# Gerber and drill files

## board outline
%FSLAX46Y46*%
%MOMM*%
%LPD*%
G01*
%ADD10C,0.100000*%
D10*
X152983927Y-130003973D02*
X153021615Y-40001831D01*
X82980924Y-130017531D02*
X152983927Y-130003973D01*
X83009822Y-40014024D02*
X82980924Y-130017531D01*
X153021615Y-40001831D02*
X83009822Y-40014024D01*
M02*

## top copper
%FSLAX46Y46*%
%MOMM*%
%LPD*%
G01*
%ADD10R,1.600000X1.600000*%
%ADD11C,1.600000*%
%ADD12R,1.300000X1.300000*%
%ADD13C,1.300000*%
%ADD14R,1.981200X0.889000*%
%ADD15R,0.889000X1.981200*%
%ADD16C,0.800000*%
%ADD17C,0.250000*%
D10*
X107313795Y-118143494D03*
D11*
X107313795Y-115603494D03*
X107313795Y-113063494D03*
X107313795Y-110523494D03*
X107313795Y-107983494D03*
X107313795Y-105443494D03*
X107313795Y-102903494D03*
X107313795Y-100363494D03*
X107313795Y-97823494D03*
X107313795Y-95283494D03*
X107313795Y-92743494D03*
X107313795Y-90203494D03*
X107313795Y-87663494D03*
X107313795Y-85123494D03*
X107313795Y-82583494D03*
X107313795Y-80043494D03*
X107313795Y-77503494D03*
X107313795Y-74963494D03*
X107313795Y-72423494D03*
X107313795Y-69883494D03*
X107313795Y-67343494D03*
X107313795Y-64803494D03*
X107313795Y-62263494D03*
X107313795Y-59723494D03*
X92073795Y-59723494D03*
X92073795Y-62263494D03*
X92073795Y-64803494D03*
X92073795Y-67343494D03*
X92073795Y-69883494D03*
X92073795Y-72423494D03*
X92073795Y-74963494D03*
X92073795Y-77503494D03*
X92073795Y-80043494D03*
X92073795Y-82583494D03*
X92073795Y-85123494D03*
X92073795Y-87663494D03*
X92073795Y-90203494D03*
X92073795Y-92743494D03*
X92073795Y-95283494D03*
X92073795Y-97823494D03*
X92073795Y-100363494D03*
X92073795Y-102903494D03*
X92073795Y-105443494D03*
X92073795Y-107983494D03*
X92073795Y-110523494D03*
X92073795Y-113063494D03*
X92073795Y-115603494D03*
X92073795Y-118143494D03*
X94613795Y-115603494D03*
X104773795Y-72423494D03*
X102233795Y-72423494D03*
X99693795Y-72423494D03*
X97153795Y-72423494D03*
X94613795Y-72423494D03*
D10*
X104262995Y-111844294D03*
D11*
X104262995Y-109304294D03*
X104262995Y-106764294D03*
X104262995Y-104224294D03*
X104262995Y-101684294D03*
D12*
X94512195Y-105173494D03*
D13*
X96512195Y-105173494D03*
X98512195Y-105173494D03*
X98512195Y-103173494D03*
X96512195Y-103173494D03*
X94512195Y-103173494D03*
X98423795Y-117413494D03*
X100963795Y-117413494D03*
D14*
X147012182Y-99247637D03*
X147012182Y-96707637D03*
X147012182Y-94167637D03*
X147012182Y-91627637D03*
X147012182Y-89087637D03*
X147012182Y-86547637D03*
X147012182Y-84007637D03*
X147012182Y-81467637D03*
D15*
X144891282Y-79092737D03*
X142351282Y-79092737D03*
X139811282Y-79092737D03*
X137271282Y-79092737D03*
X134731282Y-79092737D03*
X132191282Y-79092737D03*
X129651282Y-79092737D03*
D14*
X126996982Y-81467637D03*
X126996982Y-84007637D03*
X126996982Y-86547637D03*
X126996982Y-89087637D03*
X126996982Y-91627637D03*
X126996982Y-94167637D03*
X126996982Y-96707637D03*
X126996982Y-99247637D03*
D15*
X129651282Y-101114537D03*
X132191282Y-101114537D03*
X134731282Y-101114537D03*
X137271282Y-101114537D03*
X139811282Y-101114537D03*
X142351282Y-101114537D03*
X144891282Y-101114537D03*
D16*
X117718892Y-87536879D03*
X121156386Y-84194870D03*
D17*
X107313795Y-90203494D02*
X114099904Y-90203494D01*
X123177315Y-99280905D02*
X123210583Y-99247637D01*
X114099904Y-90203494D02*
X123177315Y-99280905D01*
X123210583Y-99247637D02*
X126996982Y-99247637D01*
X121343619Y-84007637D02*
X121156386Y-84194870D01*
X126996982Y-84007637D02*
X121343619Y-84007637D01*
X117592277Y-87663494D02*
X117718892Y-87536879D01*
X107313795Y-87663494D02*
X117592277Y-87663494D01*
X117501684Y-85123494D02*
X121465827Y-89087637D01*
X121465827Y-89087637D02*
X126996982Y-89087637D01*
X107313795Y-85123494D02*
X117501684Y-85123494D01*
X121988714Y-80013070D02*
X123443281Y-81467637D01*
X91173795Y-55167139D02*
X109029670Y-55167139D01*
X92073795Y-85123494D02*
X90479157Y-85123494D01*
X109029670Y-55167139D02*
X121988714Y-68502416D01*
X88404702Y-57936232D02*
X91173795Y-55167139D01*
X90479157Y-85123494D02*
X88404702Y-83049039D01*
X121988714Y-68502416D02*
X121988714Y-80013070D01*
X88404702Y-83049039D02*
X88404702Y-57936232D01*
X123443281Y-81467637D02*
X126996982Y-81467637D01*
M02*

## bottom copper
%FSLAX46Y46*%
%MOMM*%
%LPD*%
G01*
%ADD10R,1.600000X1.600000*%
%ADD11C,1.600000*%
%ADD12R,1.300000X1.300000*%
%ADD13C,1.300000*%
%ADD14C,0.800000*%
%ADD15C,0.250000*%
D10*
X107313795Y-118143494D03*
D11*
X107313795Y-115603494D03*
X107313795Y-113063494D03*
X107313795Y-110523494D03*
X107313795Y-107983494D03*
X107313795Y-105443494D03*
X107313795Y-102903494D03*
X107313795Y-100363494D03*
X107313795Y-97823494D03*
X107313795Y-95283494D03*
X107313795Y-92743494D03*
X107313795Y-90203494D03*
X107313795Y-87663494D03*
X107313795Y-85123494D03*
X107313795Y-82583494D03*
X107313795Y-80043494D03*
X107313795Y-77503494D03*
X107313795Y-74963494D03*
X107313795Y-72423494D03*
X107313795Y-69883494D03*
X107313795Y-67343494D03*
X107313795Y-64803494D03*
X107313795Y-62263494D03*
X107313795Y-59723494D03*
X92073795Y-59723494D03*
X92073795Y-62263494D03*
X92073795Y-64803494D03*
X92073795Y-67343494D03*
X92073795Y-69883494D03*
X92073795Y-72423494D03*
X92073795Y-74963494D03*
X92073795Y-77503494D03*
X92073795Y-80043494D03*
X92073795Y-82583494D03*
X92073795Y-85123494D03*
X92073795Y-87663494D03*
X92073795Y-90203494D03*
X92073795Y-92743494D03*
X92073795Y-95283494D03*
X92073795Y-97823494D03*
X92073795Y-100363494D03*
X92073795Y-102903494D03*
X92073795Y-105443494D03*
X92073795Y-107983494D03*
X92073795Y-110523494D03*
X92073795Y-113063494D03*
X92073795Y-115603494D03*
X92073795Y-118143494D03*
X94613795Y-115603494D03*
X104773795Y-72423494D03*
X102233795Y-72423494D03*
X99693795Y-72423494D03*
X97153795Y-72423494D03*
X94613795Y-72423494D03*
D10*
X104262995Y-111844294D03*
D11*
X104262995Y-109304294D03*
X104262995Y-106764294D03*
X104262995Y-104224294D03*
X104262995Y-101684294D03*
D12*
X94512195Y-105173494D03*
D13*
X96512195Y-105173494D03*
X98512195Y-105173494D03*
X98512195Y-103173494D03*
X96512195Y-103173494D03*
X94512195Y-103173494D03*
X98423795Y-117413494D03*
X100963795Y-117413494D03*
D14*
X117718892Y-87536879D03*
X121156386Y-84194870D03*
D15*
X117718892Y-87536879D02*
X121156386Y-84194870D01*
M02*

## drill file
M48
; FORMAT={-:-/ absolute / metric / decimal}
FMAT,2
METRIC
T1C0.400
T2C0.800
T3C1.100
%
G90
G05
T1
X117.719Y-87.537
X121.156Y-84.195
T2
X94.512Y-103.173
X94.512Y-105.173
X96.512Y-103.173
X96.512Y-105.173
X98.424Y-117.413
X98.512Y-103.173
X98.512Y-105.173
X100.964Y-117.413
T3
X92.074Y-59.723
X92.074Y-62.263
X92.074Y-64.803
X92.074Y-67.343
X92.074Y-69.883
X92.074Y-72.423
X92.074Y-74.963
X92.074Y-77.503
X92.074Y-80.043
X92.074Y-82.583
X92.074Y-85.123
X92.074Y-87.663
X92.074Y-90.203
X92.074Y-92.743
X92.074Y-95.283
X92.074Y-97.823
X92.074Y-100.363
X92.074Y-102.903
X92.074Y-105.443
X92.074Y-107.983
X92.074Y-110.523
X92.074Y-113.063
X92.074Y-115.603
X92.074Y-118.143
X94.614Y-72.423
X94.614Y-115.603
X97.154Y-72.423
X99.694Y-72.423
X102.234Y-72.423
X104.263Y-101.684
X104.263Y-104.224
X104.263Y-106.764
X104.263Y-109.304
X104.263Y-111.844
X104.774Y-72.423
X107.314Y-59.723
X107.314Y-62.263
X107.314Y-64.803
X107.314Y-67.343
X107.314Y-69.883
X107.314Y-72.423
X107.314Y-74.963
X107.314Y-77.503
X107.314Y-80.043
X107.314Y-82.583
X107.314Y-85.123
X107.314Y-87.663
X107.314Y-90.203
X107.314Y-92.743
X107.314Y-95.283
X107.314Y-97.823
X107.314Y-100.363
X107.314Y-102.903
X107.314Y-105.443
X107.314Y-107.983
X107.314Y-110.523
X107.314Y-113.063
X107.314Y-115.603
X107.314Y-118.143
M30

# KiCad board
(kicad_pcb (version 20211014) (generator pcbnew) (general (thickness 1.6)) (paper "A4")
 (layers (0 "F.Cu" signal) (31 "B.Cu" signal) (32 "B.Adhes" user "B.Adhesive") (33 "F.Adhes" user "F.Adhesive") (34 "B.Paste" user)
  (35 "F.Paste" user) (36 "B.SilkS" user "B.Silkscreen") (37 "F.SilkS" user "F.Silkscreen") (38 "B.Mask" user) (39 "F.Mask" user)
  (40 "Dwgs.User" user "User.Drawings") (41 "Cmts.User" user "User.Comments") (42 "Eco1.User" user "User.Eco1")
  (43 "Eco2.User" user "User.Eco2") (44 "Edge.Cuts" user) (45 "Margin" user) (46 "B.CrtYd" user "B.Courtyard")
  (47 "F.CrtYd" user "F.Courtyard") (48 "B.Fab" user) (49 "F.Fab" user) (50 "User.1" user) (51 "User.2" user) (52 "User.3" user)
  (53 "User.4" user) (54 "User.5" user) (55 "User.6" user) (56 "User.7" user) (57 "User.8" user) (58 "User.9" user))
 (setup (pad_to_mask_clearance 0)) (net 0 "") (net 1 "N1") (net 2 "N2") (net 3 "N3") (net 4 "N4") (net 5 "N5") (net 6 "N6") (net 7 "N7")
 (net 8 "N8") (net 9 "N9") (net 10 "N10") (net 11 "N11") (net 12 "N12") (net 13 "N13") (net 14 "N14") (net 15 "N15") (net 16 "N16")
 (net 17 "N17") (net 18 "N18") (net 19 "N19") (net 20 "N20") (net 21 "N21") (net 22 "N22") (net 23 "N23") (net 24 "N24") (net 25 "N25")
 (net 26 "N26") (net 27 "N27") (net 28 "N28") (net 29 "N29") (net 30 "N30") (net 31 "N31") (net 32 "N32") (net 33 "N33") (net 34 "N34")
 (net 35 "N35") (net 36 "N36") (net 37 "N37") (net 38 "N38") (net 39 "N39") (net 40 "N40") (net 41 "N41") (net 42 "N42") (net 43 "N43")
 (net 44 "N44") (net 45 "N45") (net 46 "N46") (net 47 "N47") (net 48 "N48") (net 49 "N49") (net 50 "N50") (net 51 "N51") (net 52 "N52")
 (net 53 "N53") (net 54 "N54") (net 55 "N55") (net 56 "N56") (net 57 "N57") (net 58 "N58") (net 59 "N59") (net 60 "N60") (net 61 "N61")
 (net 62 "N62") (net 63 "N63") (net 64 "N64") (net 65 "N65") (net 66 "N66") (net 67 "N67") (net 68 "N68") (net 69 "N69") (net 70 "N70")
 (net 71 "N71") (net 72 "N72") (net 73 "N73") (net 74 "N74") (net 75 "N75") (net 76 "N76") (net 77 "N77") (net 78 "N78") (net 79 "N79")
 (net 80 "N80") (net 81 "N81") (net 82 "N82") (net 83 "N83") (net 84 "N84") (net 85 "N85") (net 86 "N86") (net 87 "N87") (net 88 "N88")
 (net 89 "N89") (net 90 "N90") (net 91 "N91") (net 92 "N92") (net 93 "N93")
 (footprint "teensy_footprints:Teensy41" (layer "F.Cu") (at 99.693795 88.933494 90)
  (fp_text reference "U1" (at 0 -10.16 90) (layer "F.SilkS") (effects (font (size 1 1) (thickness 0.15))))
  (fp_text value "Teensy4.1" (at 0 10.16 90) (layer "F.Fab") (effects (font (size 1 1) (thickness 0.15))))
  (pad "1" thru_hole rect (at -29.21 7.62 90) (size 1.6 1.6) (drill 1.1) (layers *.Cu *.Mask) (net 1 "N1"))
  (pad "2" thru_hole circle (at -26.67 7.62 90) (size 1.6 1.6) (drill 1.1) (layers *.Cu *.Mask) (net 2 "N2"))
  (pad "3" thru_hole circle (at -24.13 7.62 90) (size 1.6 1.6) (drill 1.1) (layers *.Cu *.Mask) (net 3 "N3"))
  (pad "4" thru_hole circle (at -21.59 7.62 90) (size 1.6 1.6) (drill 1.1) (layers *.Cu *.Mask) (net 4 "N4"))
  (pad "5" thru_hole circle (at -19.05 7.62 90) (size 1.6 1.6) (drill 1.1) (layers *.Cu *.Mask) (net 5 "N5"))
  (pad "6" thru_hole circle (at -16.51 7.62 90) (size 1.6 1.6) (drill 1.1) (layers *.Cu *.Mask) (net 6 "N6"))
  (pad "7" thru_hole circle (at -13.97 7.62 90) (size 1.6 1.6) (drill 1.1) (layers *.Cu *.Mask) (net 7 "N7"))
  (pad "8" thru_hole circle (at -11.43 7.62 90) (size 1.6 1.6) (drill 1.1) (layers *.Cu *.Mask) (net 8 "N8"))
  (pad "9" thru_hole circle (at -8.89 7.62 90) (size 1.6 1.6) (drill 1.1) (layers *.Cu *.Mask) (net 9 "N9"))
  (pad "10" thru_hole circle (at -6.35 7.62 90) (size 1.6 1.6) (drill 1.1) (layers *.Cu *.Mask) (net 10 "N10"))
  (pad "11" thru_hole circle (at -3.81 7.62 90) (size 1.6 1.6) (drill 1.1) (layers *.Cu *.Mask) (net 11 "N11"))
  (pad "12" thru_hole circle (at -1.27 7.62 90) (size 1.6 1.6) (drill 1.1) (layers *.Cu *.Mask) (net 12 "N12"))
  (pad "13" thru_hole circle (at 1.27 7.62 90) (size 1.6 1.6) (drill 1.1) (layers *.Cu *.Mask) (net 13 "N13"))
  (pad "14" thru_hole circle (at 3.81 7.62 90) (size 1.6 1.6) (drill 1.1) (layers *.Cu *.Mask) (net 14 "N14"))
  (pad "15" thru_hole circle (at 6.35 7.62 90) (size 1.6 1.6) (drill 1.1) (layers *.Cu *.Mask) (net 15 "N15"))
  (pad "16" thru_hole circle (at 8.89 7.62 90) (size 1.6 1.6) (drill 1.1) (layers *.Cu *.Mask) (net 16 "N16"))
  (pad "17" thru_hole circle (at 11.43 7.62 90) (size 1.6 1.6) (drill 1.1) (layers *.Cu *.Mask) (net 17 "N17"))
  (pad "18" thru_hole circle (at 13.97 7.62 90) (size 1.6 1.6) (drill 1.1) (layers *.Cu *.Mask) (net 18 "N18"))
  (pad "19" thru_hole circle (at 16.51 7.62 90) (size 1.6 1.6) (drill 1.1) (layers *.Cu *.Mask) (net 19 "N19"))
  (pad "20" thru_hole circle (at 19.05 7.62 90) (size 1.6 1.6) (drill 1.1) (layers *.Cu *.Mask) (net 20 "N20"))
  (pad "21" thru_hole circle (at 21.59 7.62 90) (size 1.6 1.6) (drill 1.1) (layers *.Cu *.Mask) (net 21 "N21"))
  (pad "22" thru_hole circle (at 24.13 7.62 90) (size 1.6 1.6) (drill 1.1) (layers *.Cu *.Mask) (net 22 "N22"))
  (pad "23" thru_hole circle (at 26.67 7.62 90) (size 1.6 1.6) (drill 1.1) (layers *.Cu *.Mask) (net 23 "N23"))
  (pad "24" thru_hole circle (at 29.21 7.62 90) (size 1.6 1.6) (drill 1.1) (layers *.Cu *.Mask) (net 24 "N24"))
  (pad "25" thru_hole circle (at 29.21 -7.62 90) (size 1.6 1.6) (drill 1.1) (layers *.Cu *.Mask) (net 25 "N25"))
  (pad "26" thru_hole circle (at 26.67 -7.62 90) (size 1.6 1.6) (drill 1.1) (layers *.Cu *.Mask) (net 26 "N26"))
  (pad "27" thru_hole circle (at 24.13 -7.62 90) (size 1.6 1.6) (drill 1.1) (layers *.Cu *.Mask) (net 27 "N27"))
  (pad "28" thru_hole circle (at 21.59 -7.62 90) (size 1.6 1.6) (drill 1.1) (layers *.Cu *.Mask) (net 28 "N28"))
  (pad "29" thru_hole circle (at 19.05 -7.62 90) (size 1.6 1.6) (drill 1.1) (layers *.Cu *.Mask) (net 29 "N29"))
  (pad "30" thru_hole circle (at 16.51 -7.62 90) (size 1.6 1.6) (drill 1.1) (layers *.Cu *.Mask) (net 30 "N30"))
  (pad "31" thru_hole circle (at 13.97 -7.62 90) (size 1.6 1.6) (drill 1.1) (layers *.Cu *.Mask) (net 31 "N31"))
  (pad "32" thru_hole circle (at 11.43 -7.62 90) (size 1.6 1.6) (drill 1.1) (layers *.Cu *.Mask) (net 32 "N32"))
  (pad "33" thru_hole circle (at 8.89 -7.62 90) (size 1.6 1.6) (drill 1.1) (layers *.Cu *.Mask) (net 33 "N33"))
  (pad "34" thru_hole circle (at 6.35 -7.62 90) (size 1.6 1.6) (drill 1.1) (layers *.Cu *.Mask) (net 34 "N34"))
  (pad "35" thru_hole circle (at 3.81 -7.62 90) (size 1.6 1.6) (drill 1.1) (layers *.Cu *.Mask) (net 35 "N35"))
  (pad "36" thru_hole circle (at 1.27 -7.62 90) (size 1.6 1.6) (drill 1.1) (layers *.Cu *.Mask) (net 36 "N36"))
  (pad "37" thru_hole circle (at -1.27 -7.62 90) (size 1.6 1.6) (drill 1.1) (layers *.Cu *.Mask) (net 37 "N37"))
  (pad "38" thru_hole circle (at -3.81 -7.62 90) (size 1.6 1.6) (drill 1.1) (layers *.Cu *.Mask) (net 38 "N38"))
  (pad "39" thru_hole circle (at -6.35 -7.62 90) (size 1.6 1.6) (drill 1.1) (layers *.Cu *.Mask) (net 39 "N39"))
  (pad "40" thru_hole circle (at -8.89 -7.62 90) (size 1.6 1.6) (drill 1.1) (layers *.Cu *.Mask) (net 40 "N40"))
  (pad "41" thru_hole circle (at -11.43 -7.62 90) (size 1.6 1.6) (drill 1.1) (layers *.Cu *.Mask) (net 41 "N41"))
  (pad "42" thru_hole circle (at -13.97 -7.62 90) (size 1.6 1.6) (drill 1.1) (layers *.Cu *.Mask) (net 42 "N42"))
  (pad "43" thru_hole circle (at -16.51 -7.62 90) (size 1.6 1.6) (drill 1.1) (layers *.Cu *.Mask) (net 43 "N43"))
  (pad "44" thru_hole circle (at -19.05 -7.62 90) (size 1.6 1.6) (drill 1.1) (layers *.Cu *.Mask) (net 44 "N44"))
  (pad "45" thru_hole circle (at -21.59 -7.62 90) (size 1.6 1.6) (drill 1.1) (layers *.Cu *.Mask) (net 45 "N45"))
  (pad "46" thru_hole circle (at -24.13 -7.62 90) (size 1.6 1.6) (drill 1.1) (layers *.Cu *.Mask) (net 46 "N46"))
  (pad "47" thru_hole circle (at -26.67 -7.62 90) (size 1.6 1.6) (drill 1.1) (layers *.Cu *.Mask) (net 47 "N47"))
  (pad "48" thru_hole circle (at -29.21 -7.62 90) (size 1.6 1.6) (drill 1.1) (layers *.Cu *.Mask) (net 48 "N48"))
  (pad "49" thru_hole circle (at -26.67 -5.08 90) (size 1.6 1.6) (drill 1.1) (layers *.Cu *.Mask) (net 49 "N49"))
  (pad "50" thru_hole circle (at 16.51 5.08 90) (size 1.6 1.6) (drill 1.1) (layers *.Cu *.Mask) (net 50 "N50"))
  (pad "51" thru_hole circle (at 16.51 2.54 90) (size 1.6 1.6) (drill 1.1) (layers *.Cu *.Mask) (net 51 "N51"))
  (pad "52" thru_hole circle (at 16.51 0 90) (size 1.6 1.6) (drill 1.1) (layers *.Cu *.Mask) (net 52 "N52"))
  (pad "53" thru_hole circle (at 16.51 -2.54 90) (size 1.6 1.6) (drill 1.1) (layers *.Cu *.Mask) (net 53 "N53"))
  (pad "54" thru_hole circle (at 16.51 -5.08 90) (size 1.6 1.6) (drill 1.1) (layers *.Cu *.Mask) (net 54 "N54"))
  (pad "55" thru_hole rect (at -22.9108 4.5692 90) (size 1.6 1.6) (drill 1.1) (layers *.Cu *.Mask) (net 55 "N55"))
  (pad "56" thru_hole circle (at -20.3708 4.5692 90) (size 1.6 1.6) (drill 1.1) (layers *.Cu *.Mask) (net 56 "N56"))
  (pad "57" thru_hole circle (at -17.8308 4.5692 90) (size 1.6 1.6) (drill 1.1) (layers *.Cu *.Mask) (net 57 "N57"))
  (pad "58" thru_hole circle (at -15.2908 4.5692 90) (size 1.6 1.6) (drill 1.1) (layers *.Cu *.Mask) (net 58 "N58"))
  (pad "59" thru_hole circle (at -12.7508 4.5692 90) (size 1.6 1.6) (drill 1.1) (layers *.Cu *.Mask) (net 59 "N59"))
  (pad "60" thru_hole rect (at -16.24 -5.1816 90) (size 1.3 1.3) (drill 0.8) (layers *.Cu *.Mask) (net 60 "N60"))
  (pad "61" thru_hole circle (at -16.24 -3.1816 90) (size 1.3 1.3) (drill 0.8) (layers *.Cu *.Mask) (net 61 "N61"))
  (pad "62" thru_hole circle (at -16.24 -1.1816 90) (size 1.3 1.3) (drill 0.8) (layers *.Cu *.Mask) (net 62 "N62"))
  (pad "63" thru_hole circle (at -14.24 -1.1816 90) (size 1.3 1.3) (drill 0.8) (layers *.Cu *.Mask) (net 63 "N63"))
  (pad "64" thru_hole circle (at -14.24 -3.1816 90) (size 1.3 1.3) (drill 0.8) (layers *.Cu *.Mask) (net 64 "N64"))
  (pad "65" thru_hole circle (at -14.24 -5.1816 90) (size 1.3 1.3) (drill 0.8) (layers *.Cu *.Mask) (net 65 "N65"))
  (pad "66" thru_hole circle (at -28.48 -1.27 90) (size 1.3 1.3) (drill 0.8) (layers *.Cu *.Mask) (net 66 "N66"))
  (pad "67" thru_hole circle (at -28.48 1.27 90) (size 1.3 1.3) (drill 0.8) (layers *.Cu *.Mask) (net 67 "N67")))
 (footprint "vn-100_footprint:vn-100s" (layer "F.Cu") (at 137.004582 90.103637)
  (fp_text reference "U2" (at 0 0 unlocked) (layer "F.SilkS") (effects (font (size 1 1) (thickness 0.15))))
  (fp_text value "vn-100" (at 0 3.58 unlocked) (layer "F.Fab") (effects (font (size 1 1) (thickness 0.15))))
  (pad "1" smd rect (at 10.0076 9.144) (size 1.9812 0.889) (layers "F.Cu" "F.Paste" "F.Mask") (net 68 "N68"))
  (pad "2" smd rect (at 10.0076 6.604) (size 1.9812 0.889) (layers "F.Cu" "F.Paste" "F.Mask") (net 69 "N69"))
  (pad "3" smd rect (at 10.0076 4.064) (size 1.9812 0.889) (layers "F.Cu" "F.Paste" "F.Mask") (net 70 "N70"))
  (pad "4" smd rect (at 10.0076 1.524) (size 1.9812 0.889) (layers "F.Cu" "F.Paste" "F.Mask") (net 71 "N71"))
  (pad "5" smd rect (at 10.0076 -1.016) (size 1.9812 0.889) (layers "F.Cu" "F.Paste" "F.Mask") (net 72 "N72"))
  (pad "6" smd rect (at 10.0076 -3.556) (size 1.9812 0.889) (layers "F.Cu" "F.Paste" "F.Mask") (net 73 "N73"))
  (pad "7" smd rect (at 10.0076 -6.096) (size 1.9812 0.889) (layers "F.Cu" "F.Paste" "F.Mask") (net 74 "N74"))
  (pad "8" smd rect (at 10.0076 -8.636) (size 1.9812 0.889) (layers "F.Cu" "F.Paste" "F.Mask") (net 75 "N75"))
  (pad "9" smd rect (at 7.8867 -11.0109 90) (size 1.9812 0.889) (layers "F.Cu" "F.Paste" "F.Mask") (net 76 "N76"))
  (pad "10" smd rect (at 5.3467 -11.0109 90) (size 1.9812 0.889) (layers "F.Cu" "F.Paste" "F.Mask") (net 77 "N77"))
  (pad "11" smd rect (at 2.8067 -11.0109 90) (size 1.9812 0.889) (layers "F.Cu" "F.Paste" "F.Mask") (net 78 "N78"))
  (pad "12" smd rect (at 0.2667 -11.0109 90) (size 1.9812 0.889) (layers "F.Cu" "F.Paste" "F.Mask") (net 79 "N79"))
  (pad "13" smd rect (at -2.2733 -11.0109 90) (size 1.9812 0.889) (layers "F.Cu" "F.Paste" "F.Mask") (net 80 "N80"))
  (pad "14" smd rect (at -4.8133 -11.0109 90) (size 1.9812 0.889) (layers "F.Cu" "F.Paste" "F.Mask") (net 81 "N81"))
  (pad "15" smd rect (at -7.3533 -11.0109 90) (size 1.9812 0.889) (layers "F.Cu" "F.Paste" "F.Mask") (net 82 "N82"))
  (pad "16" smd rect (at -10.0076 -8.636 180) (size 1.9812 0.889) (layers "F.Cu" "F.Paste" "F.Mask") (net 35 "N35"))
  (pad "17" smd rect (at -10.0076 -6.096 180) (size 1.9812 0.889) (layers "F.Cu" "F.Paste" "F.Mask") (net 13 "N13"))
  (pad "18" smd rect (at -10.0076 -3.556 180) (size 1.9812 0.889) (layers "F.Cu" "F.Paste" "F.Mask") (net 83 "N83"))
  (pad "19" smd rect (at -10.0076 -1.016 180) (size 1.9812 0.889) (layers "F.Cu" "F.Paste" "F.Mask") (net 14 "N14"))
  (pad "20" smd rect (at -10.0076 1.524 180) (size 1.9812 0.889) (layers "F.Cu" "F.Paste" "F.Mask") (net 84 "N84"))
  (pad "21" smd rect (at -10.0076 4.064 180) (size 1.9812 0.889) (layers "F.Cu" "F.Paste" "F.Mask") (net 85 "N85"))
  (pad "22" smd rect (at -10.0076 6.604 180) (size 1.9812 0.889) (layers "F.Cu" "F.Paste" "F.Mask") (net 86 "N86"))
  (pad "23" smd rect (at -10.0076 9.144 180) (size 1.9812 0.889) (layers "F.Cu" "F.Paste" "F.Mask") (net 12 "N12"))
  (pad "24" smd rect (at -7.3533 11.0109 270) (size 1.9812 0.889) (layers "F.Cu" "F.Paste" "F.Mask") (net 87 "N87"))
  (pad "25" smd rect (at -4.8133 11.0109 270) (size 1.9812 0.889) (layers "F.Cu" "F.Paste" "F.Mask") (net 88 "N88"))
  (pad "26" smd rect (at -2.2733 11.0109 270) (size 1.9812 0.889) (layers "F.Cu" "F.Paste" "F.Mask") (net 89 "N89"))
  (pad "27" smd rect (at 0.2667 11.0109 270) (size 1.9812 0.889) (layers "F.Cu" "F.Paste" "F.Mask") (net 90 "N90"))
  (pad "28" smd rect (at 2.8067 11.0109 270) (size 1.9812 0.889) (layers "F.Cu" "F.Paste" "F.Mask") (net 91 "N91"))
  (pad "29" smd rect (at 5.3467 11.0109 270) (size 1.9812 0.889) (layers "F.Cu" "F.Paste" "F.Mask") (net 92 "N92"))
  (pad "30" smd rect (at 7.8867 11.0109 270) (size 1.9812 0.889) (layers "F.Cu" "F.Paste" "F.Mask") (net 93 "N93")))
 (gr_line (start 152.983927 130.003973) (end 153.021615 40.001831) (layer "Edge.Cuts") (width 0.1))
 (gr_line (start 82.980924 130.017531) (end 152.983927 130.003973) (layer "Edge.Cuts") (width 0.1))
 (gr_line (start 83.009822 40.014024) (end 82.980924 130.017531) (layer "Edge.Cuts") (width 0.1))
 (gr_line (start 153.021615 40.001831) (end 83.009822 40.014024) (layer "Edge.Cuts") (width 0.1))
 (segment (start 107.313795 90.203494) (end 114.099904 90.203494) (width 0.25) (layer "F.Cu") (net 12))
 (segment (start 123.177315 99.280905) (end 123.210583 99.247637) (width 0.25) (layer "F.Cu") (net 12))
 (segment (start 114.099904 90.203494) (end 123.177315 99.280905) (width 0.25) (layer "F.Cu") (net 12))
 (segment (start 123.210583 99.247637) (end 126.996982 99.247637) (width 0.25) (layer "F.Cu") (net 12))
 (segment (start 121.343619 84.007637) (end 121.156386 84.19487) (width 0.25) (layer "F.Cu") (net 13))
 (segment (start 126.996982 84.007637) (end 121.343619 84.007637) (width 0.25) (layer "F.Cu") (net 13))
 (segment (start 117.592277 87.663494) (end 117.718892 87.536879) (width 0.25) (layer "F.Cu") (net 13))
 (segment (start 107.313795 87.663494) (end 117.592277 87.663494) (width 0.25) (layer "F.Cu") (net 13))
 (via (at 117.718892 87.536879) (size 0.8) (drill 0.4) (layers "F.Cu" "B.Cu") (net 13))
 (via (at 121.156386 84.19487) (size 0.8) (drill 0.4) (layers "F.Cu" "B.Cu") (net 13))
 (segment (start 117.718892 87.536879) (end 121.156386 84.19487) (width 0.25) (layer "B.Cu") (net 13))
 (segment (start 117.501684 85.123494) (end 121.465827 89.087637) (width 0.25) (layer "F.Cu") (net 14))
 (segment (start 121.465827 89.087637) (end 126.996982 89.087637) (width 0.25) (layer "F.Cu") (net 14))
 (segment (start 107.313795 85.123494) (end 117.501684 85.123494) (width 0.25) (layer "F.Cu") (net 14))
 (segment (start 121.988714 80.01307) (end 123.443281 81.467637) (width 0.25) (layer "F.Cu") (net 35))
 (segment (start 91.173795 55.167139) (end 109.02967 55.167139) (width 0.25) (layer "F.Cu") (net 35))
 (segment (start 92.073795 85.123494) (end 90.479157 85.123494) (width 0.25) (layer "F.Cu") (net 35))
 (segment (start 109.02967 55.167139) (end 121.988714 68.502416) (width 0.25) (layer "F.Cu") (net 35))
 (segment (start 88.404702 57.936232) (end 91.173795 55.167139) (width 0.25) (layer "F.Cu") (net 35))
 (segment (start 90.479157 85.123494) (end 88.404702 83.049039) (width 0.25) (layer "F.Cu") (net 35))
 (segment (start 121.988714 68.502416) (end 121.988714 80.01307) (width 0.25) (layer "F.Cu") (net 35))
 (segment (start 88.404702 83.049039) (end 88.404702 57.936232) (width 0.25) (layer "F.Cu") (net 35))
 (segment (start 123.443281 81.467637) (end 126.996982 81.467637) (width 0.25) (layer "F.Cu") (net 35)))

